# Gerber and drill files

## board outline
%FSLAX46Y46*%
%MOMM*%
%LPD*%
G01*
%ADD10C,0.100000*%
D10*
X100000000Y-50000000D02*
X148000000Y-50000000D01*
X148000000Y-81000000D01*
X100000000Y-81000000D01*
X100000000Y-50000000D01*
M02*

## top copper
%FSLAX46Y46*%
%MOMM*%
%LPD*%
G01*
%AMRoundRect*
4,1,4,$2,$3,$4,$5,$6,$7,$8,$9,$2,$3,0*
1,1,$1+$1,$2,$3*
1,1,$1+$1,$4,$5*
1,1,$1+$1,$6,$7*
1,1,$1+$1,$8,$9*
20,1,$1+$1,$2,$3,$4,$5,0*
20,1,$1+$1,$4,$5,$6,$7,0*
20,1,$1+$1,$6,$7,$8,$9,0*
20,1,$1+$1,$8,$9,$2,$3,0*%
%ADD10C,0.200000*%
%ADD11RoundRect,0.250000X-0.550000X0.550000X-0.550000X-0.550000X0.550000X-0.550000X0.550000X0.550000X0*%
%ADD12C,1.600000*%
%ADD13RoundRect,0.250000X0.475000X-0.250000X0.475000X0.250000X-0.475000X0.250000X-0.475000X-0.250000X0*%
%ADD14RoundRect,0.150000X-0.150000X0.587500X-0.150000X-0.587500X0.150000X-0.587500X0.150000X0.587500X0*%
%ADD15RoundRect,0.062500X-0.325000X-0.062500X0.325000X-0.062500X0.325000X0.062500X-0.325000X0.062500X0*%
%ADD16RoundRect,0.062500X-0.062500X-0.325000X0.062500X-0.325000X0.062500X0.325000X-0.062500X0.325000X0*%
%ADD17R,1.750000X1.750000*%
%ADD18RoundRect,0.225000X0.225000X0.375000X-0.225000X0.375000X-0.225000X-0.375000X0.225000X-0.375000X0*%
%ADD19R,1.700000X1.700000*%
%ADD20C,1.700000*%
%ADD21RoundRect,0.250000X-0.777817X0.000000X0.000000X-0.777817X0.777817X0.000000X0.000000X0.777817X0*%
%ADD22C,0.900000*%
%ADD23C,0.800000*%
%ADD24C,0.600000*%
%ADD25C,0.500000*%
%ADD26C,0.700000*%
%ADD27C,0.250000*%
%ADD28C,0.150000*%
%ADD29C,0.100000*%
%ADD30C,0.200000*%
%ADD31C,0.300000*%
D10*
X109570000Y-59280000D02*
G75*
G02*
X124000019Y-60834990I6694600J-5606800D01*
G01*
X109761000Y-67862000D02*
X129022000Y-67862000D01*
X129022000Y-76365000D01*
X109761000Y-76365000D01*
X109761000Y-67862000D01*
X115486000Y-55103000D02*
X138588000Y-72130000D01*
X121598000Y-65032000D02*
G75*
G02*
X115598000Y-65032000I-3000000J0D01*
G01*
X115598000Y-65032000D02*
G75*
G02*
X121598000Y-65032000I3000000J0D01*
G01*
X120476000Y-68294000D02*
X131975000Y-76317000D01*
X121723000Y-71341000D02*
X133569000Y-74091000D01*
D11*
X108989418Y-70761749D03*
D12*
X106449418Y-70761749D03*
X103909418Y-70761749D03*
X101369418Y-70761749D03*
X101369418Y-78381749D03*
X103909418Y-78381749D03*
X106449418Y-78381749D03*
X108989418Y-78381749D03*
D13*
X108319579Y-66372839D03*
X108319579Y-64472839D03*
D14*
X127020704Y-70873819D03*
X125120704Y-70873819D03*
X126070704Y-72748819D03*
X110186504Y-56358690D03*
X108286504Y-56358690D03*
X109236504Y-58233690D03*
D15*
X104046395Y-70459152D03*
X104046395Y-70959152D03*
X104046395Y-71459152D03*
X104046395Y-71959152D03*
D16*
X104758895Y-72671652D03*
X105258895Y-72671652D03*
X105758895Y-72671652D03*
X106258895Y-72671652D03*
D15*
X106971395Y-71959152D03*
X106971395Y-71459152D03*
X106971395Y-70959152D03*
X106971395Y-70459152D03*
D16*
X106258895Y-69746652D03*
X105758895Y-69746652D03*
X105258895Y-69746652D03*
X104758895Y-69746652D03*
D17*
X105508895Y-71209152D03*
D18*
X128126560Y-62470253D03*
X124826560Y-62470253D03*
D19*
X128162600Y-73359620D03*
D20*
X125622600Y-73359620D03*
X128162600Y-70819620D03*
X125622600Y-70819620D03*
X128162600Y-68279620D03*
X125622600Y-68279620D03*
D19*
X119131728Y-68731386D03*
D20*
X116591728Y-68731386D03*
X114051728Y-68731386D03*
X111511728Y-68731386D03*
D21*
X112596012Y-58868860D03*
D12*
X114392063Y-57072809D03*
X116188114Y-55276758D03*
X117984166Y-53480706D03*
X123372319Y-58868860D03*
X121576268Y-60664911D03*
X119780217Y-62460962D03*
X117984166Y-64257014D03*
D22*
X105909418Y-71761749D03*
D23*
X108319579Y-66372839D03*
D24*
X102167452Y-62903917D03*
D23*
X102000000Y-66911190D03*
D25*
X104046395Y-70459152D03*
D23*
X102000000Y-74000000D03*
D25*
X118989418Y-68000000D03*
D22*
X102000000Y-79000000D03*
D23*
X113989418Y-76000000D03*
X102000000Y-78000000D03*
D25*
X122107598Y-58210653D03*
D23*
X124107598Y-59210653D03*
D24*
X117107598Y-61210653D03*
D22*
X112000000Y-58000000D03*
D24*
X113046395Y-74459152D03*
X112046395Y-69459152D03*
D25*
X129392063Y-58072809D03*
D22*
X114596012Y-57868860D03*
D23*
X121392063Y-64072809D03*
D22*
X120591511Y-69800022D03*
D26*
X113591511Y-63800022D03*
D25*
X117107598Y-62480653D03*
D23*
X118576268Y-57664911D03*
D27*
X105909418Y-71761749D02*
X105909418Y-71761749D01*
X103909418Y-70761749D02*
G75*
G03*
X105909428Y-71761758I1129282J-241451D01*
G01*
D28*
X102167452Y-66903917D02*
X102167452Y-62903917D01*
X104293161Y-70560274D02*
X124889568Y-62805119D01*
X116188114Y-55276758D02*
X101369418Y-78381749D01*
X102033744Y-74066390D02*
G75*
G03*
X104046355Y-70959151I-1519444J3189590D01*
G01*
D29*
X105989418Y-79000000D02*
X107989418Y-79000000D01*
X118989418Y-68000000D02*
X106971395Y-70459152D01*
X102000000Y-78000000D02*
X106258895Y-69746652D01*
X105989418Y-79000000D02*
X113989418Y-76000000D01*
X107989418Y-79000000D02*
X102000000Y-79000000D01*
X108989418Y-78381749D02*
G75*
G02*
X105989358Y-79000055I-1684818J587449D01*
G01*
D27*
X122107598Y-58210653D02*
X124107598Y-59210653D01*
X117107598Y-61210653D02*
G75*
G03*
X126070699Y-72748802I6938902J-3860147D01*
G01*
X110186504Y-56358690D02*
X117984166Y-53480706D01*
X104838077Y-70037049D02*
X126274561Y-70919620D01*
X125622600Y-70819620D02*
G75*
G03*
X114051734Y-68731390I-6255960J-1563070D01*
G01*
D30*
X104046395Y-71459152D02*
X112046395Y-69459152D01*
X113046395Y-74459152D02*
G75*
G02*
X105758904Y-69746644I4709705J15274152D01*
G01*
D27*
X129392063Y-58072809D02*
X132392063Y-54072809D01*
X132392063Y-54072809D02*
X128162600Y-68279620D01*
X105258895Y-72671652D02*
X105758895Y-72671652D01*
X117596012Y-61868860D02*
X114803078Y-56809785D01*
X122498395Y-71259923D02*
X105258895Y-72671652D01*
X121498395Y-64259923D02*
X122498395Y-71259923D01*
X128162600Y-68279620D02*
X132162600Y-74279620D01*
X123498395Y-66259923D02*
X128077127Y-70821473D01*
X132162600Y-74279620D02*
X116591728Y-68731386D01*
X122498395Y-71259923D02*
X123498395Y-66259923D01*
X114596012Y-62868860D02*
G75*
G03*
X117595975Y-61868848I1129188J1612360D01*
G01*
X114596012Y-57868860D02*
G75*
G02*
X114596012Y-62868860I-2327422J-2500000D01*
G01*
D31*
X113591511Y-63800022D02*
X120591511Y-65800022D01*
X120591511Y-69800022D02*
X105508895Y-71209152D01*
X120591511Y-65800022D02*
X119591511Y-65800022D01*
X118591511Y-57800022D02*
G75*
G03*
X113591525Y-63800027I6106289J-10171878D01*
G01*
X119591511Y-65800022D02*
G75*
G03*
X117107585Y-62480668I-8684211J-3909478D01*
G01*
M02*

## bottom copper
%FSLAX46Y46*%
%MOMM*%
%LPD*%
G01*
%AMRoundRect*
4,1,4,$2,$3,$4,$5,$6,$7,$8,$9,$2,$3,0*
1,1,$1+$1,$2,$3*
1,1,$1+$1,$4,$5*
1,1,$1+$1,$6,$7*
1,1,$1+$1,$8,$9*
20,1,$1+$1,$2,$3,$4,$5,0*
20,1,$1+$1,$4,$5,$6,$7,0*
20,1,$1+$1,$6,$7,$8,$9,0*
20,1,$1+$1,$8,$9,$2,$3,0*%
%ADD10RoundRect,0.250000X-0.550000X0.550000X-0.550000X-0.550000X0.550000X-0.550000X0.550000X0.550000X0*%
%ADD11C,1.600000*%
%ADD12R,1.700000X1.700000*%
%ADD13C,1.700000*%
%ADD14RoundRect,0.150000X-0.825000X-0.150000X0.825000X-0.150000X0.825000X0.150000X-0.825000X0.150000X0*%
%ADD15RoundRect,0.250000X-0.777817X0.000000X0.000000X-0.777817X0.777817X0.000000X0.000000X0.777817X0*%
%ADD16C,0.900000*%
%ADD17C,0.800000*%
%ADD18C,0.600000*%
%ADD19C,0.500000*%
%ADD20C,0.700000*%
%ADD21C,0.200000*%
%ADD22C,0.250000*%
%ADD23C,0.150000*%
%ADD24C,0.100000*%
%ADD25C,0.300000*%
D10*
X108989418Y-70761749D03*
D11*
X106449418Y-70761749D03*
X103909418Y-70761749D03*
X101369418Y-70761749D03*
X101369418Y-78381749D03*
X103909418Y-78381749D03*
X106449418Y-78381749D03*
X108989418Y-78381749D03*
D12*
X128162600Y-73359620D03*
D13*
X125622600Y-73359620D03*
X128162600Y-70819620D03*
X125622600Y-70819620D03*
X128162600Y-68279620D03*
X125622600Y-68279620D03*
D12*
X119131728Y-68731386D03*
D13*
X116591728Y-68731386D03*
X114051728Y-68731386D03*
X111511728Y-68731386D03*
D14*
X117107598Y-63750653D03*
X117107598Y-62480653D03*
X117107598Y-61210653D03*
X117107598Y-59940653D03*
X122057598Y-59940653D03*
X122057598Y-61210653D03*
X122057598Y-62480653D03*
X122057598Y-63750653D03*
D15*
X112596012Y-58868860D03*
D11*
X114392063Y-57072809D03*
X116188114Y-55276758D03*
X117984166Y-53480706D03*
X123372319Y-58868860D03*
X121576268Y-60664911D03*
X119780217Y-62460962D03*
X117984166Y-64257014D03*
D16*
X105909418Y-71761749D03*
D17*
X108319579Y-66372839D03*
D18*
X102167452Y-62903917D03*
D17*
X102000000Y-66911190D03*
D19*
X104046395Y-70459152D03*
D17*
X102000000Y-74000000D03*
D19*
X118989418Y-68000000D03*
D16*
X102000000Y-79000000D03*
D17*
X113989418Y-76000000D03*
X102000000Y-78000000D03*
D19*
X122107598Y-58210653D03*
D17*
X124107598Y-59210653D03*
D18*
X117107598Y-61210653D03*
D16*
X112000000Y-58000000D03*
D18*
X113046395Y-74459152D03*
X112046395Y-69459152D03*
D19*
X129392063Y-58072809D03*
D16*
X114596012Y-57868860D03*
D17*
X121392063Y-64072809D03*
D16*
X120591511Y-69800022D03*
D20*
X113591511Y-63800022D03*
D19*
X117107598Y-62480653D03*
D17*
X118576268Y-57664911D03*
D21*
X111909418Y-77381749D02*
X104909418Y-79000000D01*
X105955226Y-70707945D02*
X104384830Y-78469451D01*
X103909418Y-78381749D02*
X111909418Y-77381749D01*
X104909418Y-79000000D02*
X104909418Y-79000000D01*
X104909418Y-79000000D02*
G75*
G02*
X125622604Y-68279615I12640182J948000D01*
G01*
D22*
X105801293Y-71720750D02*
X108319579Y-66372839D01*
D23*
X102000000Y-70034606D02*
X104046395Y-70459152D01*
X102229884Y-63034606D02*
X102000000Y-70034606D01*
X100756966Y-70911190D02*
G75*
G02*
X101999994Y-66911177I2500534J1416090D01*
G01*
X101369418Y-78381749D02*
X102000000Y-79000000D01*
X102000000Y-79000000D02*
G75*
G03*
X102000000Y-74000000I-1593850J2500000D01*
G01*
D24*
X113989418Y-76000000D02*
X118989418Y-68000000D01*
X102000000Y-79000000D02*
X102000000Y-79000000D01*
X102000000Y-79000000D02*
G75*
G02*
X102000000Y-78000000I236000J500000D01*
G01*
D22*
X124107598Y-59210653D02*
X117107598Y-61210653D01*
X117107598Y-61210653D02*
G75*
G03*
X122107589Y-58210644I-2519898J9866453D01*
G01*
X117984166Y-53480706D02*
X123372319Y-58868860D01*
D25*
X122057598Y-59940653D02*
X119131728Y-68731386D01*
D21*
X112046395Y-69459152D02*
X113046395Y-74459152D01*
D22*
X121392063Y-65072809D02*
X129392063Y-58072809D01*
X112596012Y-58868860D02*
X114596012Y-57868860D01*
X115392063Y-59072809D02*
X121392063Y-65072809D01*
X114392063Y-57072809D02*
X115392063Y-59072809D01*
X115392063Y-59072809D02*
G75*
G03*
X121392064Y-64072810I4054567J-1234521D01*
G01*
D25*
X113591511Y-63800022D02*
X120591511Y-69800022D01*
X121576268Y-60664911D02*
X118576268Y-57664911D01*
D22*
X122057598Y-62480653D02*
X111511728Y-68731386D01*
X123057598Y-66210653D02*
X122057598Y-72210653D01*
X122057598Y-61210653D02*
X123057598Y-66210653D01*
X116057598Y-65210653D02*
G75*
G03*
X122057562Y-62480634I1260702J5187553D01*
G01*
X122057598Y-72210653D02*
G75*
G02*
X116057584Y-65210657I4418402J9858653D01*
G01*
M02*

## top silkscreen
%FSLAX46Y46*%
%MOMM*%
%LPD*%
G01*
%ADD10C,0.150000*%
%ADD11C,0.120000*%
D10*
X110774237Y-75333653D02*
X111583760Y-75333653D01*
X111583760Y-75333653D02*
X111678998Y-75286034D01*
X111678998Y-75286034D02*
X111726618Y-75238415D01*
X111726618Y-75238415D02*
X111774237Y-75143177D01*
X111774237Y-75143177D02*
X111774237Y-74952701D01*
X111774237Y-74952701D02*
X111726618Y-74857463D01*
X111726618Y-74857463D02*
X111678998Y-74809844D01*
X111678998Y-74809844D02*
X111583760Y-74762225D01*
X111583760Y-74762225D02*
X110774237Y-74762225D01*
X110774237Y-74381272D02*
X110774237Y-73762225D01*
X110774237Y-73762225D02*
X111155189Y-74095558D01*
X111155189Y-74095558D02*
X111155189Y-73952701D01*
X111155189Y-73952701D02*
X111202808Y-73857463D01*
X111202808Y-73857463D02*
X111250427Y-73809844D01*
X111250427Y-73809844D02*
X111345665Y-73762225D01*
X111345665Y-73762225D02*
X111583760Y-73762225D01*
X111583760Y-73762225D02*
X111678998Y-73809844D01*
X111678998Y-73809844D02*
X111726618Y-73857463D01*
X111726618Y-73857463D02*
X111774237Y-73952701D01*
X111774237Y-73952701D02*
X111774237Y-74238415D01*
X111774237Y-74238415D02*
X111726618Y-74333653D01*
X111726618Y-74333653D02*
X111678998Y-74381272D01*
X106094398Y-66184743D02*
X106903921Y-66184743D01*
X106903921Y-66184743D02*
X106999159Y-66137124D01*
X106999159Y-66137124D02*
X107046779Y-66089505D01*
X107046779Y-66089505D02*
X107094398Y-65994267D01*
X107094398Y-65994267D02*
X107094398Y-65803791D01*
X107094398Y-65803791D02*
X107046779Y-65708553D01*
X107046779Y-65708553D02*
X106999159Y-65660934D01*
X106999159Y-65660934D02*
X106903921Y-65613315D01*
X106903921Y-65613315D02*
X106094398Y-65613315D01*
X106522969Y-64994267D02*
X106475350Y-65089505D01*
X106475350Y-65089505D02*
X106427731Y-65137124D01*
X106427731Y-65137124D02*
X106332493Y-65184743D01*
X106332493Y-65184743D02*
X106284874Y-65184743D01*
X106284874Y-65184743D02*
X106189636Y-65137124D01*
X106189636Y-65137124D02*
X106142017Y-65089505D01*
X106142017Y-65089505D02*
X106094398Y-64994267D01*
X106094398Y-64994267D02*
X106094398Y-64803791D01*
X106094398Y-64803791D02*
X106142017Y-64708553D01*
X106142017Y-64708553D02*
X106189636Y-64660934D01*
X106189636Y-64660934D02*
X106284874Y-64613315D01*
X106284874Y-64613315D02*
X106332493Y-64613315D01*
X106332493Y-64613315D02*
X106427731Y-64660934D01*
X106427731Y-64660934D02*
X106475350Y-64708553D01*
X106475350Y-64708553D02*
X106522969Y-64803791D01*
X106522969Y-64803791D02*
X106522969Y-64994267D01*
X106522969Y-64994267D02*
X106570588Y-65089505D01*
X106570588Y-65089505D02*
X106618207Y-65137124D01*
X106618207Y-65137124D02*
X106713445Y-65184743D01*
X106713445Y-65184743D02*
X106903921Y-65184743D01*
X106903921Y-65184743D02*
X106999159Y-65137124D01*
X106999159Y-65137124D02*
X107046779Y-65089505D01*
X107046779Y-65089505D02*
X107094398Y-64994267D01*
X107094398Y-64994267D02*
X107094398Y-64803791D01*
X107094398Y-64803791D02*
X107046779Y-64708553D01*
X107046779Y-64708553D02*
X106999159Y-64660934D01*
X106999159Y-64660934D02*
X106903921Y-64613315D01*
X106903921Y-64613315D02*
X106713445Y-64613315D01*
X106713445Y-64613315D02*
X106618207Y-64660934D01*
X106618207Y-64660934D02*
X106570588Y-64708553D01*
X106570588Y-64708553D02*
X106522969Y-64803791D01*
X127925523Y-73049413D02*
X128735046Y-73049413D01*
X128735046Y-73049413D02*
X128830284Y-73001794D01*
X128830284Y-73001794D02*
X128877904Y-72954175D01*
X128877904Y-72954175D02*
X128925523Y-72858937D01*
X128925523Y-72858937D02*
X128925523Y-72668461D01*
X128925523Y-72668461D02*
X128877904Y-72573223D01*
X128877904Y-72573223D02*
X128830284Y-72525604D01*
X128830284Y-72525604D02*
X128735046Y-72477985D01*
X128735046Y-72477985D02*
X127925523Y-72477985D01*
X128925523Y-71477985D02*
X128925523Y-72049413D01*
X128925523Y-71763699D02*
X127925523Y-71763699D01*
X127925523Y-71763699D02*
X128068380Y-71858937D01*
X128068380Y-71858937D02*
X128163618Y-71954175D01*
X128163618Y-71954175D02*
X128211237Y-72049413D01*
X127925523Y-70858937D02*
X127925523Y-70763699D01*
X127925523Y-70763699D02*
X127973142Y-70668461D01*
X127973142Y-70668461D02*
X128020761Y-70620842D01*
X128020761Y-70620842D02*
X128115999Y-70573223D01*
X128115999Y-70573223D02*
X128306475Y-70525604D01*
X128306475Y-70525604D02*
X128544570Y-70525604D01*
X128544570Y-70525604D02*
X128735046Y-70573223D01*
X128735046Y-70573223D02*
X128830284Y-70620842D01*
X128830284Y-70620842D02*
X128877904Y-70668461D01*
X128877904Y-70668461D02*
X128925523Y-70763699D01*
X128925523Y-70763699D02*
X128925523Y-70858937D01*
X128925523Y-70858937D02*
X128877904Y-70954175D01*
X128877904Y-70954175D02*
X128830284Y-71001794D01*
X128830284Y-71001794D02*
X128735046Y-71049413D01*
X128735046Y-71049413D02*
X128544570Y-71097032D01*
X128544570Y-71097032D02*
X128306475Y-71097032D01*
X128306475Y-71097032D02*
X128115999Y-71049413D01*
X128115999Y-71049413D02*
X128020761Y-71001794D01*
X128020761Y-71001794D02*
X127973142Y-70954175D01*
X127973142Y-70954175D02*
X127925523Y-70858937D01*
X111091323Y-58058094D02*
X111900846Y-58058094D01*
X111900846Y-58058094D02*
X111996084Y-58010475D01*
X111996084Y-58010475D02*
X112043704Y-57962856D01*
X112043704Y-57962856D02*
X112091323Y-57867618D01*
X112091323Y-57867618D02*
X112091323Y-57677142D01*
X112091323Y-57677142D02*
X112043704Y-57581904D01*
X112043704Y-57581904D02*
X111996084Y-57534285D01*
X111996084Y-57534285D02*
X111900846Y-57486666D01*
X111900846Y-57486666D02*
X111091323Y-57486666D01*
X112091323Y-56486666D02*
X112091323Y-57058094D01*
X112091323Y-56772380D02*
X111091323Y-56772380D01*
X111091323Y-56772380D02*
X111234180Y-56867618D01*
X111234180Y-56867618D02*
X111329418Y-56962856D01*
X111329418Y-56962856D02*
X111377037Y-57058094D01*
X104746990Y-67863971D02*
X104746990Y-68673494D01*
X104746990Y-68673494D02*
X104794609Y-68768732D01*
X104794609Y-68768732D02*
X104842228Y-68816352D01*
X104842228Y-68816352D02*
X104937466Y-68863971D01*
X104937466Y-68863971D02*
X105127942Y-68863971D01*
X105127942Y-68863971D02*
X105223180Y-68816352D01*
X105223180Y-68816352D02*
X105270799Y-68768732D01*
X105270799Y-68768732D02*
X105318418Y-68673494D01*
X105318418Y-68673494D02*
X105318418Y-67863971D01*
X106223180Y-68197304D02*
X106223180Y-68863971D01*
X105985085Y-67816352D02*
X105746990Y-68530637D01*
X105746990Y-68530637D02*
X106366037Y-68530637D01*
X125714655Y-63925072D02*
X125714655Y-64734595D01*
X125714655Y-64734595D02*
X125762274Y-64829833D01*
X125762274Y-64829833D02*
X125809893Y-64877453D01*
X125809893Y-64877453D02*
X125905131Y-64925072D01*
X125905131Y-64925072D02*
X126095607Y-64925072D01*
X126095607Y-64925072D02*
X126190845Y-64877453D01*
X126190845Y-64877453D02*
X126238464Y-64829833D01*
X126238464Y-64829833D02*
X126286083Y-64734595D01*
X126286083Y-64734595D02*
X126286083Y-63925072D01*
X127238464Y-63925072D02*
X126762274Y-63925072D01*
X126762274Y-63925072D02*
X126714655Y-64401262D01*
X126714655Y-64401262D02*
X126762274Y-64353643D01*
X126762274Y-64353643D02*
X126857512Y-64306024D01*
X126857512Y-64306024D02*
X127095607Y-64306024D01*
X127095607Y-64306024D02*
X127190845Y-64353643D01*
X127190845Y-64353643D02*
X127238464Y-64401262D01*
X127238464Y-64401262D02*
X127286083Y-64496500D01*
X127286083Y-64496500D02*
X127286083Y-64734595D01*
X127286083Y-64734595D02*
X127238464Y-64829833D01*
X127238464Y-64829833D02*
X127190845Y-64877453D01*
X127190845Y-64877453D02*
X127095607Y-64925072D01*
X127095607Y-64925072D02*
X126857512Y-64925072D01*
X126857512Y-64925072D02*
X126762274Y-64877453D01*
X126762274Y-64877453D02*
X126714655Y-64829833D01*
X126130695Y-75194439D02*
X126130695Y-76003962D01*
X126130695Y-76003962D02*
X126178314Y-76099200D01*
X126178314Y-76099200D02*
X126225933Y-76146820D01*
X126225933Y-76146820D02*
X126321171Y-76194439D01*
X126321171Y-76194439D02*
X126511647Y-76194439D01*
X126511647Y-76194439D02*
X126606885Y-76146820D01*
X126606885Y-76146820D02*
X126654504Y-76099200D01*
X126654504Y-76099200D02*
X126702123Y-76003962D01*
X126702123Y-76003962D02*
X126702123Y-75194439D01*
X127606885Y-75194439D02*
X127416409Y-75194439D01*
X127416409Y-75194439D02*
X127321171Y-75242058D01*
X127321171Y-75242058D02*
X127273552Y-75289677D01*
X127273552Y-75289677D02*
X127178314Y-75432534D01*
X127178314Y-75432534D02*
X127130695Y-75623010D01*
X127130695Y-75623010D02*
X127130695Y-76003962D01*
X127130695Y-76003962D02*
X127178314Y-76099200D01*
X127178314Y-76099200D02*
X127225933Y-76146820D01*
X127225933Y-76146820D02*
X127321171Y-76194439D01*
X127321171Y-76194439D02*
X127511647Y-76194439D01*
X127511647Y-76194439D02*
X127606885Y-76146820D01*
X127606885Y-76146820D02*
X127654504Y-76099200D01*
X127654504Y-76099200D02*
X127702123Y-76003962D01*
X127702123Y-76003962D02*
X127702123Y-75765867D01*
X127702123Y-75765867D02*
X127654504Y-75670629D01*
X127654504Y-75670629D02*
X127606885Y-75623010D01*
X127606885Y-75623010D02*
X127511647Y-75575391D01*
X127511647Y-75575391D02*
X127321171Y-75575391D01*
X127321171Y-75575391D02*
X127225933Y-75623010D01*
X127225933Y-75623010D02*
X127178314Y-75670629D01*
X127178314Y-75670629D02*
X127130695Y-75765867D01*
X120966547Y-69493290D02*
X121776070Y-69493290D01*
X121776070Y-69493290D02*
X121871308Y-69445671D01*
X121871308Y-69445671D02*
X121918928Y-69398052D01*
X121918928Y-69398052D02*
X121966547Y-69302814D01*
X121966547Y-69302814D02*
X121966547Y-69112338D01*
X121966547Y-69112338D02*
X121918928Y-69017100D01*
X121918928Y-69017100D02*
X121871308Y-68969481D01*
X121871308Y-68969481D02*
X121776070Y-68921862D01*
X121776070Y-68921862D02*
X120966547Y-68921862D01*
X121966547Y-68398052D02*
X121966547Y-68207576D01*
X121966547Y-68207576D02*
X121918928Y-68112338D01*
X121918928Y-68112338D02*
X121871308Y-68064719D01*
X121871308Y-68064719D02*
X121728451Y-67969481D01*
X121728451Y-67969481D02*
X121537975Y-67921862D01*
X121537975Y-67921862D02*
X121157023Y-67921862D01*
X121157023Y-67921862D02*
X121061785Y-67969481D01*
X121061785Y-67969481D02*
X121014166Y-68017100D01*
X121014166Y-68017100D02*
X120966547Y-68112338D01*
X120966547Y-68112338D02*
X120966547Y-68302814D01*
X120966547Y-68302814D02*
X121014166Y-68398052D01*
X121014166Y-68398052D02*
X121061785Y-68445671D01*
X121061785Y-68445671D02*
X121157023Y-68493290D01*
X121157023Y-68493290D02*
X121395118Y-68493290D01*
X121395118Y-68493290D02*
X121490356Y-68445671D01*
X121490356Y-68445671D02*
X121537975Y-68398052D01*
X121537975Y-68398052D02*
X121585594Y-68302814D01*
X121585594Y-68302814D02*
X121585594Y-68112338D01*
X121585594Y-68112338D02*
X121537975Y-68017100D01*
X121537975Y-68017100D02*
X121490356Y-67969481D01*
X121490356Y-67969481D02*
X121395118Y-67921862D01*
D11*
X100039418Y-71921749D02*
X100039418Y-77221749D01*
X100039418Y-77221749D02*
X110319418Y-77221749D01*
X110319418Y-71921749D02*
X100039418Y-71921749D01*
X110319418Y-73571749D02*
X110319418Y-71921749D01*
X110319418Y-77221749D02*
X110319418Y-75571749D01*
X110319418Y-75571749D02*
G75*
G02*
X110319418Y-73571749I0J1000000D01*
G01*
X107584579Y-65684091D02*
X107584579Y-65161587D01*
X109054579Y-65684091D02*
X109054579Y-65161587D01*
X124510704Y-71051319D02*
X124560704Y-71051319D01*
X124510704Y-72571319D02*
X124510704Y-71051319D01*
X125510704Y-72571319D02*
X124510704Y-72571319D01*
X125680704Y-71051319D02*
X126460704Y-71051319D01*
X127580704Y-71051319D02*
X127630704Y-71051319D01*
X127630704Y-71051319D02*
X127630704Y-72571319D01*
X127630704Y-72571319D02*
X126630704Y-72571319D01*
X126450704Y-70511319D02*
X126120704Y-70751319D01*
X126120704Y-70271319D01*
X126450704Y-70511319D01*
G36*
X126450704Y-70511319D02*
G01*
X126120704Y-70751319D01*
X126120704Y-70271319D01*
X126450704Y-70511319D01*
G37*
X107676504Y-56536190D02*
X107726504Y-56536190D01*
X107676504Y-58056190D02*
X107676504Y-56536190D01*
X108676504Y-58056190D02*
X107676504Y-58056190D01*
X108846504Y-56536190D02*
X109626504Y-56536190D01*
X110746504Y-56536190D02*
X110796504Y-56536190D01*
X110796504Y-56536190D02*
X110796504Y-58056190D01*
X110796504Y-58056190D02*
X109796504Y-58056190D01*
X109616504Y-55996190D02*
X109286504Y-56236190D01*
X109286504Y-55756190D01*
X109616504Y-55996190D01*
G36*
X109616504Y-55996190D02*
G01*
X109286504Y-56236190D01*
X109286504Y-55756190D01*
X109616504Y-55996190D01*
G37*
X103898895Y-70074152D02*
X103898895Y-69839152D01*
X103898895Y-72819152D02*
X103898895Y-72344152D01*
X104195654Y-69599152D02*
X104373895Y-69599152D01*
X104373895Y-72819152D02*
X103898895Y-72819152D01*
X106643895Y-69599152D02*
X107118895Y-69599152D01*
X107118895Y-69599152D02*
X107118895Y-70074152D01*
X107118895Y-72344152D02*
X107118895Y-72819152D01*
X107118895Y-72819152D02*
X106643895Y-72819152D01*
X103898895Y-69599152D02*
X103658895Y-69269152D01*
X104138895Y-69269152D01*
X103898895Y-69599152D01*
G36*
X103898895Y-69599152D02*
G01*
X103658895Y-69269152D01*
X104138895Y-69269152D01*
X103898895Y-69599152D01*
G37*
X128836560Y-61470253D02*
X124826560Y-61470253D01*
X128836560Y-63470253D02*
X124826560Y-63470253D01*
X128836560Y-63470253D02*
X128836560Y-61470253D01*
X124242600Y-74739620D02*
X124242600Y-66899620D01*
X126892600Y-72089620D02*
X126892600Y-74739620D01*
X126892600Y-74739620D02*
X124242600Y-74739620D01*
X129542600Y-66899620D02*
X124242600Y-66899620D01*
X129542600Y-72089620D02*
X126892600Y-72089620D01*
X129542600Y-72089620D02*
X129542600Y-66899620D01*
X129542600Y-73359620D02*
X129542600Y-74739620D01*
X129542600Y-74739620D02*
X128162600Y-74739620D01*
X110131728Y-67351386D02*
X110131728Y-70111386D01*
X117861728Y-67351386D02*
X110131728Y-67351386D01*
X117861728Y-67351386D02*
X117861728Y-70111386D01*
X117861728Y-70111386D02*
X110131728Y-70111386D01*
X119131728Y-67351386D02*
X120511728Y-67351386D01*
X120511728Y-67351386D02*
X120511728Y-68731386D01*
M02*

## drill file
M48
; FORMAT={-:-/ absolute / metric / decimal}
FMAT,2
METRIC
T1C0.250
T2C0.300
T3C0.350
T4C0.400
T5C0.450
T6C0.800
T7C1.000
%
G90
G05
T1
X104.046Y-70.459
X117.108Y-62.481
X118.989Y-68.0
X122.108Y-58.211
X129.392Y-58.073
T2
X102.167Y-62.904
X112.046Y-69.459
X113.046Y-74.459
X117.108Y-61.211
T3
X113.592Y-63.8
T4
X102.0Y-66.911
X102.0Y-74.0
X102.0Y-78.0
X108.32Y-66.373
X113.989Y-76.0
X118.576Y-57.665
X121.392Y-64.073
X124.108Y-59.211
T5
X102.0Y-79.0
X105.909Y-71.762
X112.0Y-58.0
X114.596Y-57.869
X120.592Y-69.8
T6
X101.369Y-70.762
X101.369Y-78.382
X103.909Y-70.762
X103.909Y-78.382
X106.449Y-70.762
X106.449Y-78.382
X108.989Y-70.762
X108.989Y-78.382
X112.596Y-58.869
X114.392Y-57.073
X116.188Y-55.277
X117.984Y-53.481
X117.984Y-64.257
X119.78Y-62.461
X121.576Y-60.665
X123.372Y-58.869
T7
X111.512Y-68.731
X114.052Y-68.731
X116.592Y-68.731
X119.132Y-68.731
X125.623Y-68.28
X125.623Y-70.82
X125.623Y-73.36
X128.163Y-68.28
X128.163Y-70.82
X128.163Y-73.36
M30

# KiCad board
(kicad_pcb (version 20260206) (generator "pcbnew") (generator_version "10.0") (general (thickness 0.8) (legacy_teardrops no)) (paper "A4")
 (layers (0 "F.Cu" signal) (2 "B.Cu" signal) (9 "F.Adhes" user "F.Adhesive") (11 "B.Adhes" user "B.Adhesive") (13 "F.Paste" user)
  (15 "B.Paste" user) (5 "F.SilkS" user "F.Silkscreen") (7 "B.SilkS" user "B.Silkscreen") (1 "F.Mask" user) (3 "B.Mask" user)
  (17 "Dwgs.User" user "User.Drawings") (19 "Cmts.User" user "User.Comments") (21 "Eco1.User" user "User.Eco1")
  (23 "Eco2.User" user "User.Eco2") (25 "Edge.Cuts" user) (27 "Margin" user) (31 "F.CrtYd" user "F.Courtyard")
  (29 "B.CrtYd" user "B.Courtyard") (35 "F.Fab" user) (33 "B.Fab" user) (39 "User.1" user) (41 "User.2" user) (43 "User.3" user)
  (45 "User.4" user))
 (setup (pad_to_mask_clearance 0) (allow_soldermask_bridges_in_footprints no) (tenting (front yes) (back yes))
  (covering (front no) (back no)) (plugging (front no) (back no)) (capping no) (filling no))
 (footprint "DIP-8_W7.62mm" (layer "F.Cu") (at 108.989418 70.761749 -90)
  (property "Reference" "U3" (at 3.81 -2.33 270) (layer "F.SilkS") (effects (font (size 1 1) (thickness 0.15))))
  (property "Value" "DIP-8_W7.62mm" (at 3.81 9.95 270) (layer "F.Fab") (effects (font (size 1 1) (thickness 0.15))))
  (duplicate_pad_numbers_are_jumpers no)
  (fp_line (start 1.16 8.95) (end 6.46 8.95) (stroke (width 0.12) (type solid)) (layer "F.SilkS"))
  (fp_line (start 6.46 8.95) (end 6.46 -1.33) (stroke (width 0.12) (type solid)) (layer "F.SilkS"))
  (fp_line (start 1.16 -1.33) (end 1.16 8.95) (stroke (width 0.12) (type solid)) (layer "F.SilkS"))
  (fp_line (start 2.81 -1.33) (end 1.16 -1.33) (stroke (width 0.12) (type solid)) (layer "F.SilkS"))
  (fp_line (start 6.46 -1.33) (end 4.81 -1.33) (stroke (width 0.12) (type solid)) (layer "F.SilkS"))
  (fp_arc (start 4.81 -1.33) (mid 3.81 -0.33) (end 2.81 -1.33) (stroke (width 0.12) (type solid)) (layer "F.SilkS"))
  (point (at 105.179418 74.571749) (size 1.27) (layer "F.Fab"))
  (pad "1" thru_hole roundrect (at 0 0 270) (size 1.6 1.6) (drill 0.8) (layers "*.Cu" "*.Mask") (remove_unused_layers no)
   (roundrect_rratio 0.15625))
  (pad "2" thru_hole circle (at 0 2.54 270) (size 1.6 1.6) (drill 0.8) (layers "*.Cu" "*.Mask") (remove_unused_layers no) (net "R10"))
  (pad "3" thru_hole circle (at 0 5.08 270) (size 1.6 1.6) (drill 0.8) (layers "*.Cu" "*.Mask") (remove_unused_layers no) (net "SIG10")
   (die_length 0.3))
  (pad "4" thru_hole circle (at 0 7.62 270) (size 1.6 1.6) (drill 0.8) (layers "*.Cu" "*.Mask") (remove_unused_layers no)
   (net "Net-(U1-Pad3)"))
  (pad "5" thru_hole circle (at 7.62 7.62 270) (size 1.6 1.6) (drill 0.8) (layers "*.Cu" "*.Mask") (remove_unused_layers no)
   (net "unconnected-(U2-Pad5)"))
  (pad "6" thru_hole circle (at 7.62 5.08 270) (size 1.6 1.6) (drill 0.8) (layers "*.Cu" "*.Mask") (remove_unused_layers no) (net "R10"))
  (pad "7" thru_hole circle (at 7.62 2.54 270) (size 1.6 1.6) (drill 0.8) (layers "*.Cu" "*.Mask") (remove_unused_layers no))
  (pad "8" thru_hole circle (at 7.62 0 270) (size 1.6 1.6) (drill 0.8) (layers "*.Cu" "*.Mask") (remove_unused_layers no) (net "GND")))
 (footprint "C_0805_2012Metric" (layer "F.Cu") (at 108.319579 65.422839 90)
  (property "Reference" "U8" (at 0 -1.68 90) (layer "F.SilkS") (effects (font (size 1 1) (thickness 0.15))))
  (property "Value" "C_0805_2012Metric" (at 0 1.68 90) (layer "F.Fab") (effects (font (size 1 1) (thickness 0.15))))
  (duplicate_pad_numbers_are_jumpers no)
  (fp_line (start -0.261252 -0.735) (end 0.261252 -0.735) (stroke (width 0.12) (type solid)) (layer "F.SilkS"))
  (fp_line (start -0.261252 0.735) (end 0.261252 0.735) (stroke (width 0.12) (type solid)) (layer "F.SilkS"))
  (pad "1" smd roundrect (at -0.95 0 90) (size 1 1.45) (layers "F.Cu" "F.Mask" "F.Paste") (roundrect_rratio 0.25) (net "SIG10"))
  (pad "2" smd roundrect (at 0.95 0 90) (size 1 1.45) (layers "F.Cu" "F.Mask" "F.Paste") (roundrect_rratio 0.25)))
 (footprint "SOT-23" (layer "F.Cu") (at 126.070704 71.811319 -90)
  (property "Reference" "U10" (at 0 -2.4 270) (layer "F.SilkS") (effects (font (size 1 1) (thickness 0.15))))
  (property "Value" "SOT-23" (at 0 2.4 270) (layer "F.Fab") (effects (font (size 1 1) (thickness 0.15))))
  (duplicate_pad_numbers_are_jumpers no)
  (fp_line (start -0.76 1.56) (end -0.76 1.51) (stroke (width 0.12) (type solid)) (layer "F.SilkS"))
  (fp_line (start 0.76 1.56) (end -0.76 1.56) (stroke (width 0.12) (type solid)) (layer "F.SilkS"))
  (fp_line (start 0.76 0.56) (end 0.76 1.56) (stroke (width 0.12) (type solid)) (layer "F.SilkS"))
  (fp_line (start -0.76 0.39) (end -0.76 -0.39) (stroke (width 0.12) (type solid)) (layer "F.SilkS"))
  (fp_line (start -0.76 -1.51) (end -0.76 -1.56) (stroke (width 0.12) (type solid)) (layer "F.SilkS"))
  (fp_line (start -0.76 -1.56) (end 0.76 -1.56) (stroke (width 0.12) (type solid)) (layer "F.SilkS"))
  (fp_line (start 0.76 -1.56) (end 0.76 -0.56) (stroke (width 0.12) (type solid)) (layer "F.SilkS"))
  (fp_poly (pts (xy -1.3 -0.38) (xy -1.06 -0.05) (xy -1.54 -0.05)) (stroke (width 0.12) (type solid)) (fill yes) (layer "F.SilkS"))
  (pad "1" smd roundrect (at -0.9375 -0.95 270) (size 1.475 0.6) (layers "F.Cu" "F.Mask" "F.Paste") (roundrect_rratio 0.25)
   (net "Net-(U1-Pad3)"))
  (pad "2" smd roundrect (at -0.9375 0.95 270) (size 1.475 0.6) (layers "F.Cu" "F.Mask" "F.Paste") (roundrect_rratio 0.25) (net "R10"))
  (pad "3" smd roundrect (at 0.9375 0 270) (size 1.475 0.6) (layers "F.Cu" "F.Mask" "F.Paste") (roundrect_rratio 0.25) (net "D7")
   (die_length 2.7)))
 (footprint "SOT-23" (layer "F.Cu") (at 109.236504 57.29619 -90)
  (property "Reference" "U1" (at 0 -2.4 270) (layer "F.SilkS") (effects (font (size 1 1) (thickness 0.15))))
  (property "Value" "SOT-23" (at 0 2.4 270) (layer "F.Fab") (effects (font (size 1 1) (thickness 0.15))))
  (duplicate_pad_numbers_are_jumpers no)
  (fp_line (start -0.76 1.56) (end -0.76 1.51) (stroke (width 0.12) (type solid)) (layer "F.SilkS"))
  (fp_line (start 0.76 1.56) (end -0.76 1.56) (stroke (width 0.12) (type solid)) (layer "F.SilkS"))
  (fp_line (start 0.76 0.56) (end 0.76 1.56) (stroke (width 0.12) (type solid)) (layer "F.SilkS"))
  (fp_line (start -0.76 0.39) (end -0.76 -0.39) (stroke (width 0.12) (type solid)) (layer "F.SilkS"))
  (fp_line (start -0.76 -1.51) (end -0.76 -1.56) (stroke (width 0.12) (type solid)) (layer "F.SilkS"))
  (fp_line (start -0.76 -1.56) (end 0.76 -1.56) (stroke (width 0.12) (type solid)) (layer "F.SilkS"))
  (fp_line (start 0.76 -1.56) (end 0.76 -0.56) (stroke (width 0.12) (type solid)) (layer "F.SilkS"))
  (fp_poly (pts (xy -1.3 -0.38) (xy -1.06 -0.05) (xy -1.54 -0.05)) (stroke (width 0.12) (type solid)) (fill yes) (layer "F.SilkS"))
  (pad "1" smd roundrect (at -0.9375 -0.95 270) (size 1.475 0.6) (layers "F.Cu" "F.Mask" "F.Paste") (roundrect_rratio 0.25) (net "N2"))
  (pad "2" smd roundrect (at -0.9375 0.95 270) (size 1.475 0.6) (layers "F.Cu" "F.Mask" "F.Paste") (roundrect_rratio 0.25))
  (pad "3" smd roundrect (at 0.9375 0 270) (size 1.475 0.6) (layers "F.Cu" "F.Mask" "F.Paste") (roundrect_rratio 0.25) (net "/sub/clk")
   (die_length 2.5)))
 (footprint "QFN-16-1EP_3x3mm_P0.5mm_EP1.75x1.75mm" (layer "F.Cu") (at 105.508895 71.209152)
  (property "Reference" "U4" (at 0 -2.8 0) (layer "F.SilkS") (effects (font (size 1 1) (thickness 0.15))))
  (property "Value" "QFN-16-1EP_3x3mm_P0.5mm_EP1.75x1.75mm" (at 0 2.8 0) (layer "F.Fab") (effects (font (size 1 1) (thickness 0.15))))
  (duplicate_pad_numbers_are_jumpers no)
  (fp_line (start -1.61 -1.135) (end -1.61 -1.37) (stroke (width 0.12) (type solid)) (layer "F.SilkS"))
  (fp_line (start -1.61 1.61) (end -1.61 1.135) (stroke (width 0.12) (type solid)) (layer "F.SilkS"))
  (fp_line (start -1.313241 -1.61) (end -1.135 -1.61) (stroke (width 0.12) (type solid)) (layer "F.SilkS"))
  (fp_line (start -1.135 1.61) (end -1.61 1.61) (stroke (width 0.12) (type solid)) (layer "F.SilkS"))
  (fp_line (start 1.135 -1.61) (end 1.61 -1.61) (stroke (width 0.12) (type solid)) (layer "F.SilkS"))
  (fp_line (start 1.61 -1.61) (end 1.61 -1.135) (stroke (width 0.12) (type solid)) (layer "F.SilkS"))
  (fp_line (start 1.61 1.135) (end 1.61 1.61) (stroke (width 0.12) (type solid)) (layer "F.SilkS"))
  (fp_line (start 1.61 1.61) (end 1.135 1.61) (stroke (width 0.12) (type solid)) (layer "F.SilkS"))
  (fp_poly (pts (xy -1.61 -1.61) (xy -1.85 -1.94) (xy -1.37 -1.94)) (stroke (width 0.12) (type solid)) (fill yes) (layer "F.SilkS"))
  (pad "" smd roundrect (at -0.44 -0.44) (size 0.71 0.71) (layers "F.Paste") (roundrect_rratio 0.25))
  (pad "" smd roundrect (at -0.44 0.44) (size 0.71 0.71) (layers "F.Paste") (roundrect_rratio 0.25) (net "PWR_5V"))
  (pad "" smd roundrect (at 0.44 -0.44) (size 0.71 0.71) (layers "F.Paste") (roundrect_rratio 0.25))
  (pad "" smd roundrect (at 0.44 0.44) (size 0.71 0.71) (layers "F.Paste") (roundrect_rratio 0.25))
  (pad "1" smd roundrect (at -1.4625 -0.75) (size 0.775 0.25) (layers "F.Cu" "F.Mask" "F.Paste") (roundrect_rratio 0.25)
   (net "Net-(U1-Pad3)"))
  (pad "2" smd roundrect (at -1.4625 -0.25) (size 0.775 0.25) (layers "F.Cu" "F.Mask" "F.Paste") (roundrect_rratio 0.25)
   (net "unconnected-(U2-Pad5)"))
  (pad "3" smd roundrect (at -1.4625 0.25) (size 0.775 0.25) (layers "F.Cu" "F.Mask" "F.Paste") (roundrect_rratio 0.25) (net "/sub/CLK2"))
  (pad "4" smd roundrect (at -1.4625 0.75) (size 0.775 0.25) (layers "F.Cu" "F.Mask" "F.Paste") (roundrect_rratio 0.25))
  (pad "5" smd roundrect (at -0.75 1.4625) (size 0.25 0.775) (layers "F.Cu" "F.Mask" "F.Paste") (roundrect_rratio 0.25) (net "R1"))
  (pad "6" smd roundrect (at -0.25 1.4625) (size 0.25 0.775) (layers "F.Cu" "F.Mask" "F.Paste") (roundrect_rratio 0.25) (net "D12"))
  (pad "7" smd roundrect (at 0.25 1.4625) (size 0.25 0.775) (layers "F.Cu" "F.Mask" "F.Paste") (roundrect_rratio 0.25) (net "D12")
   (die_length 3.3))
  (pad "8" smd roundrect (at 0.75 1.4625) (size 0.25 0.775) (layers "F.Cu" "F.Mask" "F.Paste") (roundrect_rratio 0.25))
  (pad "9" smd roundrect (at 1.4625 0.75) (size 0.775 0.25) (layers "F.Cu" "F.Mask" "F.Paste") (roundrect_rratio 0.25))
  (pad "10" smd roundrect (at 1.4625 0.25) (size 0.775 0.25) (layers "F.Cu" "F.Mask" "F.Paste") (roundrect_rratio 0.25))
  (pad "11" smd roundrect (at 1.4625 -0.25) (size 0.775 0.25) (layers "F.Cu" "F.Mask" "F.Paste") (roundrect_rratio 0.25))
  (pad "12" smd roundrect (at 1.4625 -0.75) (size 0.775 0.25) (layers "F.Cu" "F.Mask" "F.Paste") (roundrect_rratio 0.25) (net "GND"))
  (pad "13" smd roundrect (at 0.75 -1.4625) (size 0.25 0.775) (layers "F.Cu" "F.Mask" "F.Paste") (roundrect_rratio 0.25) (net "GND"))
  (pad "14" smd roundrect (at 0.25 -1.4625) (size 0.25 0.775) (layers "F.Cu" "F.Mask" "F.Paste") (roundrect_rratio 0.25) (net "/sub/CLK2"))
  (pad "15" smd roundrect (at -0.25 -1.4625) (size 0.25 0.775) (layers "F.Cu" "F.Mask" "F.Paste") (roundrect_rratio 0.25))
  (pad "16" smd roundrect (at -0.75 -1.4625) (size 0.25 0.775) (layers "F.Cu" "F.Mask" "F.Paste") (roundrect_rratio 0.25) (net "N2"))
  (pad "17" smd rect (at 0 0) (size 1.75 1.75) (layers "F.Cu" "F.Mask") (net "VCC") (zone_connect 2)))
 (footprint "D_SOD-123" (layer "F.Cu") (at 126.47656 62.470253 180)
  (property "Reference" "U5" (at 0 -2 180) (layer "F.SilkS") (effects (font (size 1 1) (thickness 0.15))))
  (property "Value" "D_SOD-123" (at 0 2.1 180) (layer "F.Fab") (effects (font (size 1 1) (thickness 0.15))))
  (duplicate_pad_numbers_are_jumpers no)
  (fp_line (start -2.36 1) (end 1.65 1) (stroke (width 0.12) (type solid)) (layer "F.SilkS"))
  (fp_line (start -2.36 -1) (end 1.65 -1) (stroke (width 0.12) (type solid)) (layer "F.SilkS"))
  (fp_line (start -2.36 -1) (end -2.36 1) (stroke (width 0.12) (type solid)) (layer "F.SilkS"))
  (pad "1" smd roundrect (at -1.65 0 180) (size 0.9 1.2) (layers "F.Cu" "F.Mask" "F.Paste") (roundrect_rratio 0.25))
  (pad "2" smd roundrect (at 1.65 0 180) (size 0.9 1.2) (layers "F.Cu" "F.Mask" "F.Paste") (roundrect_rratio 0.25) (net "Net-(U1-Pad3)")))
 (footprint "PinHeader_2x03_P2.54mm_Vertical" (layer "F.Cu") (at 128.1626 73.35962 180)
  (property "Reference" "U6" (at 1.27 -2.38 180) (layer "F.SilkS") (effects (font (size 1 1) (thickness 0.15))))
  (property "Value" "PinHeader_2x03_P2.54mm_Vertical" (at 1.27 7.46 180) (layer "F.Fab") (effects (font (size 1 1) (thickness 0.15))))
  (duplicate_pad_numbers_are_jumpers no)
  (fp_line (start 3.92 -1.38) (end 3.92 6.46) (stroke (width 0.12) (type solid)) (layer "F.SilkS"))
  (fp_line (start 1.27 1.27) (end 1.27 -1.38) (stroke (width 0.12) (type solid)) (layer "F.SilkS"))
  (fp_line (start 1.27 -1.38) (end 3.92 -1.38) (stroke (width 0.12) (type solid)) (layer "F.SilkS"))
  (fp_line (start -1.38 6.46) (end 3.92 6.46) (stroke (width 0.12) (type solid)) (layer "F.SilkS"))
  (fp_line (start -1.38 1.27) (end 1.27 1.27) (stroke (width 0.12) (type solid)) (layer "F.SilkS"))
  (fp_line (start -1.38 1.27) (end -1.38 6.46) (stroke (width 0.12) (type solid)) (layer "F.SilkS"))
  (fp_line (start -1.38 0) (end -1.38 -1.38) (stroke (width 0.12) (type solid)) (layer "F.SilkS"))
  (fp_line (start -1.38 -1.38) (end 0 -1.38) (stroke (width 0.12) (type solid)) (layer "F.SilkS"))
  (pad "1" thru_hole rect (at 0 0 180) (size 1.7 1.7) (drill 1) (layers "*.Cu" "*.Mask") (remove_unused_layers no) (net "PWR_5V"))
  (pad "2" thru_hole circle (at 2.54 0 180) (size 1.7 1.7) (drill 1) (layers "*.Cu" "*.Mask") (remove_unused_layers no))
  (pad "3" thru_hole circle (at 0 2.54 180) (size 1.7 1.7) (drill 1) (layers "*.Cu" "*.Mask") (remove_unused_layers no) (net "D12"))
  (pad "4" thru_hole circle (at 2.54 2.54 180) (size 1.7 1.7) (drill 1) (layers "*.Cu" "*.Mask") (remove_unused_layers no) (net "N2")
   (die_length 0.1))
  (pad "5" thru_hole circle (at 0 5.08 180) (size 1.7 1.7) (drill 1) (layers "*.Cu" "*.Mask") (remove_unused_layers no) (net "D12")
   (die_length 2.7))
  (pad "6" thru_hole circle (at 2.54 5.08 180) (size 1.7 1.7) (drill 1) (layers "*.Cu" "*.Mask") (remove_unused_layers no) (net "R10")
   (die_length 0.6)))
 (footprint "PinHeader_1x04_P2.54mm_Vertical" (layer "F.Cu") (at 119.131728 68.731386 -90)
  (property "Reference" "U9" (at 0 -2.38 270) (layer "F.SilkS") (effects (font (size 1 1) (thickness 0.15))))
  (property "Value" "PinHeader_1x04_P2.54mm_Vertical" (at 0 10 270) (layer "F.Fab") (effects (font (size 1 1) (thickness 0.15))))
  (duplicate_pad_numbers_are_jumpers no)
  (fp_line (start -1.38 9) (end 1.38 9) (stroke (width 0.12) (type solid)) (layer "F.SilkS"))
  (fp_line (start -1.38 1.27) (end -1.38 9) (stroke (width 0.12) (type solid)) (layer "F.SilkS"))
  (fp_line (start -1.38 1.27) (end 1.38 1.27) (stroke (width 0.12) (type solid)) (layer "F.SilkS"))
  (fp_line (start 1.38 1.27) (end 1.38 9) (stroke (width 0.12) (type solid)) (layer "F.SilkS"))
  (fp_line (start -1.38 0) (end -1.38 -1.38) (stroke (width 0.12) (type solid)) (layer "F.SilkS"))
  (fp_line (start -1.38 -1.38) (end 0 -1.38) (stroke (width 0.12) (type solid)) (layer "F.SilkS"))
  (pad "1" thru_hole rect (at 0 0 270) (size 1.7 1.7) (drill 1) (layers "*.Cu" "*.Mask") (remove_unused_layers no) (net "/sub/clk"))
  (pad "2" thru_hole circle (at 0 2.54 270) (size 1.7 1.7) (drill 1) (layers "*.Cu" "*.Mask") (remove_unused_layers no) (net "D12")
   (die_length 4.4))
  (pad "3" thru_hole circle (at 0 5.08 270) (size 1.7 1.7) (drill 1) (layers "*.Cu" "*.Mask") (remove_unused_layers no) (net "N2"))
  (pad "4" thru_hole circle (at 0 7.62 270) (size 1.7 1.7) (drill 1) (layers "*.Cu" "*.Mask") (remove_unused_layers no) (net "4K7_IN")))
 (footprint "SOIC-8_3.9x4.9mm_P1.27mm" (layer "B.Cu") (at 119.582598 61.845653)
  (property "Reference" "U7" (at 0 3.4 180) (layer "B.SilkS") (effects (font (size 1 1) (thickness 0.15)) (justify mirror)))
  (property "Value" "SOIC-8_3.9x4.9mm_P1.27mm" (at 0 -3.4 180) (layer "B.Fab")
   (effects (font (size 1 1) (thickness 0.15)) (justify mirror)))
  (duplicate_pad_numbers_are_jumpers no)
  (pad "1" smd roundrect (at -2.475 1.905) (size 1.95 0.6) (layers "B.Cu" "B.Mask" "B.Paste") (roundrect_rratio 0.25))
  (pad "2" smd roundrect (at -2.475 0.635) (size 1.95 0.6) (layers "B.Cu" "B.Mask" "B.Paste") (roundrect_rratio 0.25) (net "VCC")
   (die_length 1.7))
  (pad "3" smd roundrect (at -2.475 -0.635) (size 1.95 0.6) (layers "B.Cu" "B.Mask" "B.Paste") (roundrect_rratio 0.25) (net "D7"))
  (pad "4" smd roundrect (at -2.475 -1.905) (size 1.95 0.6) (layers "B.Cu" "B.Mask" "B.Paste") (roundrect_rratio 0.25) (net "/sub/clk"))
  (pad "5" smd roundrect (at 2.475 -1.905) (size 1.95 0.6) (layers "B.Cu" "B.Mask" "B.Paste") (roundrect_rratio 0.25) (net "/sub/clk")
   (die_length 1.6))
  (pad "6" smd roundrect (at 2.475 -0.635) (size 1.95 0.6) (layers "B.Cu" "B.Mask" "B.Paste") (roundrect_rratio 0.25) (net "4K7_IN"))
  (pad "7" smd roundrect (at 2.475 0.635) (size 1.95 0.6) (layers "B.Cu" "B.Mask" "B.Paste") (roundrect_rratio 0.25) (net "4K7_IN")
   (die_length 3.2))
  (pad "8" smd roundrect (at 2.475 1.905) (size 1.95 0.6) (layers "B.Cu" "B.Mask" "B.Paste") (roundrect_rratio 0.25)))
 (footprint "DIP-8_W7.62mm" (layer "B.Cu") (at 112.596012 58.86886 -45)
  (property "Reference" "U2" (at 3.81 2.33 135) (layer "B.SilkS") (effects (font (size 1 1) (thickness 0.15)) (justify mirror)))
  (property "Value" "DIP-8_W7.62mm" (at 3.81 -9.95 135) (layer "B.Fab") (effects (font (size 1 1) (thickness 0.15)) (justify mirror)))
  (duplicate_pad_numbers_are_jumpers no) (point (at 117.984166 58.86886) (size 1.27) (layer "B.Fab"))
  (pad "1" thru_hole roundrect (at 0 0 315) (size 1.6 1.6) (drill 0.8) (layers "*.Cu" "*.Mask") (remove_unused_layers no)
   (roundrect_rratio 0.15625) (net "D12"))
  (pad "2" thru_hole circle (at 0 -2.54 315) (size 1.6 1.6) (drill 0.8) (layers "*.Cu" "*.Mask") (remove_unused_layers no) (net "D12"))
  (pad "3" thru_hole circle (at 0 -5.079999 315) (size 1.6 1.6) (drill 0.8) (layers "*.Cu" "*.Mask") (remove_unused_layers no)
   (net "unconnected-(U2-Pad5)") (die_length 4.5))
  (pad "4" thru_hole circle (at 0 -7.62 315) (size 1.6 1.6) (drill 0.8) (layers "*.Cu" "*.Mask") (remove_unused_layers no) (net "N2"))
  (pad "5" thru_hole circle (at 7.62 -7.62 315) (size 1.6 1.6) (drill 0.8) (layers "*.Cu" "*.Mask") (remove_unused_layers no) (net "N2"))
  (pad "6" thru_hole circle (at 7.62 -5.08 315) (size 1.6 1.6) (drill 0.8) (layers "*.Cu" "*.Mask") (remove_unused_layers no) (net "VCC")
   (die_length 1.5))
  (pad "7" thru_hole circle (at 7.62 -2.54 315) (size 1.6 1.6) (drill 0.8) (layers "*.Cu" "*.Mask") (remove_unused_layers no)
   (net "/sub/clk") (die_length 1.6))
  (pad "8" thru_hole circle (at 7.62 0 315) (size 1.6 1.6) (drill 0.8) (layers "*.Cu" "*.Mask") (remove_unused_layers no)))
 (gr_arc (start 109.57 59.28) (mid 116.785 56.17) (end 124 60.835) (stroke (width 0.2) (type default)) (layer "F.Cu"))
 (gr_rect (start 109.761 67.862) (end 129.022 76.365) (stroke (width 0.2) (type default)) (fill no) (layer "F.Cu"))
 (gr_line (start 115.486 55.103) (end 138.588 72.13) (stroke (width 0.2) (type default)) (layer "F.Cu"))
 (gr_circle (center 118.598 65.032) (end 121.598 65.032) (stroke (width 0.2) (type default)) (fill no) (layer "F.Cu"))
 (gr_line (start 120.476 68.294) (end 131.975 76.317) (stroke (width 0.2) (type default)) (layer "F.Cu"))
 (gr_line (start 121.723 71.341) (end 133.569 74.091) (stroke (width 0.2) (type default)) (layer "F.Cu"))
 (gr_rect (start 100 50) (end 148 81) (stroke (width 0.1) (type default)) (fill no) (layer "Edge.Cuts"))
 (segment (start 111.909418 77.381749) (end 104.909418 79) (width 0.2) (layer "B.Cu") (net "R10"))
 (segment (start 105.955226 70.707945) (end 104.38483 78.469451) (width 0.2) (layer "B.Cu") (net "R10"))
 (segment (start 103.909418 78.381749) (end 111.909418 77.381749) (width 0.2) (layer "B.Cu") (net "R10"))
 (segment (start 104.909418 79) (end 104.909418 79) (width 0.2) (layer "B.Cu") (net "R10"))
 (arc (start 104.909418 79) (mid 111.72324 66.794716) (end 125.6226 68.27962) (width 0.2) (layer "B.Cu") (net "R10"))
 (segment (start 105.909418 71.761749) (end 105.909418 71.761749) (width 0.25) (layer "F.Cu") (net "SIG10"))
 (via (at 105.909418 71.761749) (size 0.9) (drill 0.45) (layers "F.Cu" "B.Cu") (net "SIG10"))
 (via (at 108.319579 66.372839) (size 0.8) (drill 0.4) (layers "F.Cu" "B.Cu") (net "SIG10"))
 (arc (start 103.909418 70.761749) (mid 104.522233 72.036117) (end 105.909418 71.761749) (width 0.25) (layer "F.Cu") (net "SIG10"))
 (segment (start 105.801293 71.72075) (end 108.319579 66.372839) (width 0.25) (layer "B.Cu") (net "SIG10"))
 (segment (start 102.167452 66.903917) (end 102.167452 62.903917) (width 0.15) (layer "F.Cu") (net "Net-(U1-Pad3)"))
 (segment (start 104.293161 70.560274) (end 124.889568 62.805119) (width 0.15) (layer "F.Cu") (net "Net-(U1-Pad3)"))
 (via (at 102.167452 62.903917) (size 0.6) (drill 0.3) (layers "F.Cu" "B.Cu") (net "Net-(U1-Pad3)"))
 (via (at 102 66.91119) (size 0.8) (drill 0.4) (layers "F.Cu" "B.Cu") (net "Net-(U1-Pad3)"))
 (via (at 104.046395 70.459152) (size 0.5) (drill 0.25) (layers "F.Cu" "B.Cu") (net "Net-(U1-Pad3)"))
 (segment (start 102 70.034606) (end 104.046395 70.459152) (width 0.15) (layer "B.Cu") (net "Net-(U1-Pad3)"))
 (segment (start 102.229884 63.034606) (end 102 70.034606) (width 0.15) (layer "B.Cu") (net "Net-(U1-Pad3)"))
 (arc (start 100.756966 70.91119) (mid 100.513273 68.642318) (end 102 66.91119) (width 0.15) (layer "B.Cu") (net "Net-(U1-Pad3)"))
 (segment (start 116.188114 55.276758) (end 101.369418 78.381749) (width 0.15) (layer "F.Cu") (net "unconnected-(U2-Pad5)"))
 (via (at 102 74) (size 0.8) (drill 0.4) (layers "F.Cu" "B.Cu") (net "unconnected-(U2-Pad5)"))
 (arc (start 102.033744 74.06639) (mid 103.479646 72.797498) (end 104.046395 70.959152) (width 0.15) (layer "F.Cu")
  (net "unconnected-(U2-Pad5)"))
 (segment (start 101.369418 78.381749) (end 102 79) (width 0.15) (layer "B.Cu") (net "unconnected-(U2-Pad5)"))
 (arc (start 102 79) (mid 103.371004 76.5) (end 102 74) (width 0.15) (layer "B.Cu") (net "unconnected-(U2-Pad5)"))
 (segment (start 105.989418 79) (end 107.989418 79) (width 0.1) (layer "F.Cu") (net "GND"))
 (segment (start 118.989418 68) (end 106.971395 70.459152) (width 0.1) (layer "F.Cu") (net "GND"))
 (segment (start 102 78) (end 106.258895 69.746652) (width 0.1) (layer "F.Cu") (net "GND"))
 (segment (start 105.989418 79) (end 113.989418 76) (width 0.1) (layer "F.Cu") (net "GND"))
 (segment (start 107.989418 79) (end 102 79) (width 0.1) (layer "F.Cu") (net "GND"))
 (via (at 118.989418 68) (size 0.5) (drill 0.25) (layers "F.Cu" "B.Cu") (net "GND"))
 (via (at 102 79) (size 0.9) (drill 0.45) (layers "F.Cu" "B.Cu") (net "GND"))
 (via (at 113.989418 76) (size 0.8) (drill 0.4) (layers "F.Cu" "B.Cu") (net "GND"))
 (via (at 102 78) (size 0.8) (drill 0.4) (layers "F.Cu" "B.Cu") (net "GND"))
 (arc (start 108.989418 78.381749) (mid 107.664785 79.541828) (end 105.989418 79) (width 0.1) (layer "F.Cu") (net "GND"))
 (segment (start 113.989418 76) (end 118.989418 68) (width 0.1) (layer "B.Cu") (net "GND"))
 (segment (start 102 79) (end 102 79) (width 0.1) (layer "B.Cu") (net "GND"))
 (arc (start 102 79) (mid 101.68312 78.5) (end 102 78) (width 0.1) (layer "B.Cu") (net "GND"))
 (segment (start 122.107598 58.210653) (end 124.107598 59.210653) (width 0.25) (layer "F.Cu") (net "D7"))
 (via (at 122.107598 58.210653) (size 0.5) (drill 0.25) (layers "F.Cu" "B.Cu") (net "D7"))
 (via (at 124.107598 59.210653) (size 0.8) (drill 0.4) (layers "F.Cu" "B.Cu") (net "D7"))
 (via (at 117.107598 61.210653) (size 0.6) (drill 0.3) (layers "F.Cu" "B.Cu") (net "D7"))
 (arc (start 117.107598 61.210653) (mid 117.775869 69.941978) (end 126.070704 72.748819) (width 0.25) (layer "F.Cu") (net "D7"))
 (segment (start 124.107598 59.210653) (end 117.107598 61.210653) (width 0.25) (layer "B.Cu") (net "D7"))
 (arc (start 117.107598 61.210653) (mid 119.826915 60.076182) (end 122.107598 58.210653) (width 0.25) (layer "B.Cu") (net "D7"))
 (segment (start 110.186504 56.35869) (end 117.984166 53.480706) (width 0.25) (layer "F.Cu") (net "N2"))
 (segment (start 104.838077 70.037049) (end 126.274561 70.91962) (width 0.25) (layer "F.Cu") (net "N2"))
 (via (at 112 58) (size 0.9) (drill 0.45) (layers "F.Cu" "B.Cu") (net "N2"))
 (arc (start 125.6226 70.81962) (mid 120.511877 66.036926) (end 114.051728 68.731386) (width 0.25) (layer "F.Cu") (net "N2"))
 (segment (start 117.984166 53.480706) (end 123.372319 58.86886) (width 0.25) (layer "B.Cu") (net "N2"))
 (segment (start 122.057598 59.940653) (end 119.131728 68.731386) (width 0.3) (layer "B.Cu") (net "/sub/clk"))
 (segment (start 104.046395 71.459152) (end 112.046395 69.459152) (width 0.2) (layer "F.Cu") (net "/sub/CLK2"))
 (via (at 113.046395 74.459152) (size 0.6) (drill 0.3) (layers "F.Cu" "B.Cu") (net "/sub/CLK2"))
 (via (at 112.046395 69.459152) (size 0.6) (drill 0.3) (layers "F.Cu" "B.Cu") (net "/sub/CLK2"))
 (arc (start 113.046395 74.459152) (mid 109.076691 72.606963) (end 105.758895 69.746652) (width 0.2) (layer "F.Cu") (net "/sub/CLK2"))
 (segment (start 112.046395 69.459152) (end 113.046395 74.459152) (width 0.2) (layer "B.Cu") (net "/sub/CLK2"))
 (segment (start 129.392063 58.072809) (end 132.392063 54.072809) (width 0.25) (layer "F.Cu") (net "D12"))
 (segment (start 132.392063 54.072809) (end 128.1626 68.27962) (width 0.25) (layer "F.Cu") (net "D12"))
 (segment (start 105.258895 72.671652) (end 105.758895 72.671652) (width 0.25) (layer "F.Cu") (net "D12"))
 (segment (start 117.596012 61.86886) (end 114.803078 56.809785) (width 0.25) (layer "F.Cu") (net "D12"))
 (segment (start 122.498395 71.259923) (end 105.258895 72.671652) (width 0.25) (layer "F.Cu") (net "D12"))
 (segment (start 121.498395 64.259923) (end 122.498395 71.259923) (width 0.25) (layer "F.Cu") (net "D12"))
 (segment (start 128.1626 68.27962) (end 132.1626 74.27962) (width 0.25) (layer "F.Cu") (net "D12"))
 (segment (start 123.498395 66.259923) (end 128.077127 70.821473) (width 0.25) (layer "F.Cu") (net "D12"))
 (segment (start 132.1626 74.27962) (end 116.591728 68.731386) (width 0.25) (layer "F.Cu") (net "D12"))
 (segment (start 122.498395 71.259923) (end 123.498395 66.259923) (width 0.25) (layer "F.Cu") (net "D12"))
 (via (at 129.392063 58.072809) (size 0.5) (drill 0.25) (layers "F.Cu" "B.Cu") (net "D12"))
 (via (at 114.596012 57.86886) (size 0.9) (drill 0.45) (layers "F.Cu" "B.Cu") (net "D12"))
 (via (at 121.392063 64.072809) (size 0.8) (drill 0.4) (layers "F.Cu" "B.Cu") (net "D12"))
 (arc (start 114.596012 62.86886) (mid 116.347708 63.123949) (end 117.596012 61.86886) (width 0.25) (layer "F.Cu") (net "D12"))
 (arc (start 114.596012 57.86886) (mid 115.684274 60.36886) (end 114.596012 62.86886) (width 0.25) (layer "F.Cu") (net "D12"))
 (segment (start 121.392063 65.072809) (end 129.392063 58.072809) (width 0.25) (layer "B.Cu") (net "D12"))
 (segment (start 112.596012 58.86886) (end 114.596012 57.86886) (width 0.25) (layer "B.Cu") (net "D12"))
 (segment (start 115.392063 59.072809) (end 121.392063 65.072809) (width 0.25) (layer "B.Cu") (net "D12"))
 (segment (start 114.392063 57.072809) (end 115.392063 59.072809) (width 0.25) (layer "B.Cu") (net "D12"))
 (arc (start 115.392063 59.072809) (mid 116.733308 63.563314) (end 121.392063 64.072809) (width 0.25) (layer "B.Cu") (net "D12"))
 (segment (start 113.591511 63.800022) (end 120.591511 65.800022) (width 0.3) (layer "F.Cu") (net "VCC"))
 (segment (start 120.591511 69.800022) (end 105.508895 71.209152) (width 0.3) (layer "F.Cu") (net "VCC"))
 (segment (start 120.591511 65.800022) (end 119.591511 65.800022) (width 0.3) (layer "F.Cu") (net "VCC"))
 (via (at 120.591511 69.800022) (size 0.9) (drill 0.45) (layers "F.Cu" "B.Cu") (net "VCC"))
 (via (at 113.591511 63.800022) (size 0.7) (drill 0.35) (layers "F.Cu" "B.Cu") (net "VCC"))
 (via (at 117.107598 62.480653) (size 0.5) (drill 0.25) (layers "F.Cu" "B.Cu") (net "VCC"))
 (via (at 118.576268 57.664911) (size 0.8) (drill 0.4) (layers "F.Cu" "B.Cu") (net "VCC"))
 (arc (start 118.591511 57.800022) (mid 115.583622 60.376781) (end 113.591511 63.800022) (width 0.3) (layer "F.Cu") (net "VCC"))
 (arc (start 119.591511 65.800022) (mid 118.53237 64.003534) (end 117.107598 62.480653) (width 0.3) (layer "F.Cu") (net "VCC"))
 (segment (start 113.591511 63.800022) (end 120.591511 69.800022) (width 0.3) (layer "B.Cu") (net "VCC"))
 (segment (start 121.576268 60.664911) (end 118.576268 57.664911) (width 0.3) (layer "B.Cu") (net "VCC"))
 (segment (start 122.057598 62.480653) (end 111.511728 68.731386) (width 0.25) (layer "B.Cu") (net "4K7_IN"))
 (segment (start 123.057598 66.210653) (end 122.057598 72.210653) (width 0.25) (layer "B.Cu") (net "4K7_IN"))
 (segment (start 122.057598 61.210653) (end 123.057598 66.210653) (width 0.25) (layer "B.Cu") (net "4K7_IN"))
 (arc (start 116.057598 65.210653) (mid 119.529277 64.88231) (end 122.057598 62.480653) (width 0.25) (layer "B.Cu") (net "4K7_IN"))
 (arc (start 122.057598 72.210653) (mid 118.273399 69.382823) (end 116.057598 65.210653) (width 0.25) (layer "B.Cu") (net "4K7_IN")))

